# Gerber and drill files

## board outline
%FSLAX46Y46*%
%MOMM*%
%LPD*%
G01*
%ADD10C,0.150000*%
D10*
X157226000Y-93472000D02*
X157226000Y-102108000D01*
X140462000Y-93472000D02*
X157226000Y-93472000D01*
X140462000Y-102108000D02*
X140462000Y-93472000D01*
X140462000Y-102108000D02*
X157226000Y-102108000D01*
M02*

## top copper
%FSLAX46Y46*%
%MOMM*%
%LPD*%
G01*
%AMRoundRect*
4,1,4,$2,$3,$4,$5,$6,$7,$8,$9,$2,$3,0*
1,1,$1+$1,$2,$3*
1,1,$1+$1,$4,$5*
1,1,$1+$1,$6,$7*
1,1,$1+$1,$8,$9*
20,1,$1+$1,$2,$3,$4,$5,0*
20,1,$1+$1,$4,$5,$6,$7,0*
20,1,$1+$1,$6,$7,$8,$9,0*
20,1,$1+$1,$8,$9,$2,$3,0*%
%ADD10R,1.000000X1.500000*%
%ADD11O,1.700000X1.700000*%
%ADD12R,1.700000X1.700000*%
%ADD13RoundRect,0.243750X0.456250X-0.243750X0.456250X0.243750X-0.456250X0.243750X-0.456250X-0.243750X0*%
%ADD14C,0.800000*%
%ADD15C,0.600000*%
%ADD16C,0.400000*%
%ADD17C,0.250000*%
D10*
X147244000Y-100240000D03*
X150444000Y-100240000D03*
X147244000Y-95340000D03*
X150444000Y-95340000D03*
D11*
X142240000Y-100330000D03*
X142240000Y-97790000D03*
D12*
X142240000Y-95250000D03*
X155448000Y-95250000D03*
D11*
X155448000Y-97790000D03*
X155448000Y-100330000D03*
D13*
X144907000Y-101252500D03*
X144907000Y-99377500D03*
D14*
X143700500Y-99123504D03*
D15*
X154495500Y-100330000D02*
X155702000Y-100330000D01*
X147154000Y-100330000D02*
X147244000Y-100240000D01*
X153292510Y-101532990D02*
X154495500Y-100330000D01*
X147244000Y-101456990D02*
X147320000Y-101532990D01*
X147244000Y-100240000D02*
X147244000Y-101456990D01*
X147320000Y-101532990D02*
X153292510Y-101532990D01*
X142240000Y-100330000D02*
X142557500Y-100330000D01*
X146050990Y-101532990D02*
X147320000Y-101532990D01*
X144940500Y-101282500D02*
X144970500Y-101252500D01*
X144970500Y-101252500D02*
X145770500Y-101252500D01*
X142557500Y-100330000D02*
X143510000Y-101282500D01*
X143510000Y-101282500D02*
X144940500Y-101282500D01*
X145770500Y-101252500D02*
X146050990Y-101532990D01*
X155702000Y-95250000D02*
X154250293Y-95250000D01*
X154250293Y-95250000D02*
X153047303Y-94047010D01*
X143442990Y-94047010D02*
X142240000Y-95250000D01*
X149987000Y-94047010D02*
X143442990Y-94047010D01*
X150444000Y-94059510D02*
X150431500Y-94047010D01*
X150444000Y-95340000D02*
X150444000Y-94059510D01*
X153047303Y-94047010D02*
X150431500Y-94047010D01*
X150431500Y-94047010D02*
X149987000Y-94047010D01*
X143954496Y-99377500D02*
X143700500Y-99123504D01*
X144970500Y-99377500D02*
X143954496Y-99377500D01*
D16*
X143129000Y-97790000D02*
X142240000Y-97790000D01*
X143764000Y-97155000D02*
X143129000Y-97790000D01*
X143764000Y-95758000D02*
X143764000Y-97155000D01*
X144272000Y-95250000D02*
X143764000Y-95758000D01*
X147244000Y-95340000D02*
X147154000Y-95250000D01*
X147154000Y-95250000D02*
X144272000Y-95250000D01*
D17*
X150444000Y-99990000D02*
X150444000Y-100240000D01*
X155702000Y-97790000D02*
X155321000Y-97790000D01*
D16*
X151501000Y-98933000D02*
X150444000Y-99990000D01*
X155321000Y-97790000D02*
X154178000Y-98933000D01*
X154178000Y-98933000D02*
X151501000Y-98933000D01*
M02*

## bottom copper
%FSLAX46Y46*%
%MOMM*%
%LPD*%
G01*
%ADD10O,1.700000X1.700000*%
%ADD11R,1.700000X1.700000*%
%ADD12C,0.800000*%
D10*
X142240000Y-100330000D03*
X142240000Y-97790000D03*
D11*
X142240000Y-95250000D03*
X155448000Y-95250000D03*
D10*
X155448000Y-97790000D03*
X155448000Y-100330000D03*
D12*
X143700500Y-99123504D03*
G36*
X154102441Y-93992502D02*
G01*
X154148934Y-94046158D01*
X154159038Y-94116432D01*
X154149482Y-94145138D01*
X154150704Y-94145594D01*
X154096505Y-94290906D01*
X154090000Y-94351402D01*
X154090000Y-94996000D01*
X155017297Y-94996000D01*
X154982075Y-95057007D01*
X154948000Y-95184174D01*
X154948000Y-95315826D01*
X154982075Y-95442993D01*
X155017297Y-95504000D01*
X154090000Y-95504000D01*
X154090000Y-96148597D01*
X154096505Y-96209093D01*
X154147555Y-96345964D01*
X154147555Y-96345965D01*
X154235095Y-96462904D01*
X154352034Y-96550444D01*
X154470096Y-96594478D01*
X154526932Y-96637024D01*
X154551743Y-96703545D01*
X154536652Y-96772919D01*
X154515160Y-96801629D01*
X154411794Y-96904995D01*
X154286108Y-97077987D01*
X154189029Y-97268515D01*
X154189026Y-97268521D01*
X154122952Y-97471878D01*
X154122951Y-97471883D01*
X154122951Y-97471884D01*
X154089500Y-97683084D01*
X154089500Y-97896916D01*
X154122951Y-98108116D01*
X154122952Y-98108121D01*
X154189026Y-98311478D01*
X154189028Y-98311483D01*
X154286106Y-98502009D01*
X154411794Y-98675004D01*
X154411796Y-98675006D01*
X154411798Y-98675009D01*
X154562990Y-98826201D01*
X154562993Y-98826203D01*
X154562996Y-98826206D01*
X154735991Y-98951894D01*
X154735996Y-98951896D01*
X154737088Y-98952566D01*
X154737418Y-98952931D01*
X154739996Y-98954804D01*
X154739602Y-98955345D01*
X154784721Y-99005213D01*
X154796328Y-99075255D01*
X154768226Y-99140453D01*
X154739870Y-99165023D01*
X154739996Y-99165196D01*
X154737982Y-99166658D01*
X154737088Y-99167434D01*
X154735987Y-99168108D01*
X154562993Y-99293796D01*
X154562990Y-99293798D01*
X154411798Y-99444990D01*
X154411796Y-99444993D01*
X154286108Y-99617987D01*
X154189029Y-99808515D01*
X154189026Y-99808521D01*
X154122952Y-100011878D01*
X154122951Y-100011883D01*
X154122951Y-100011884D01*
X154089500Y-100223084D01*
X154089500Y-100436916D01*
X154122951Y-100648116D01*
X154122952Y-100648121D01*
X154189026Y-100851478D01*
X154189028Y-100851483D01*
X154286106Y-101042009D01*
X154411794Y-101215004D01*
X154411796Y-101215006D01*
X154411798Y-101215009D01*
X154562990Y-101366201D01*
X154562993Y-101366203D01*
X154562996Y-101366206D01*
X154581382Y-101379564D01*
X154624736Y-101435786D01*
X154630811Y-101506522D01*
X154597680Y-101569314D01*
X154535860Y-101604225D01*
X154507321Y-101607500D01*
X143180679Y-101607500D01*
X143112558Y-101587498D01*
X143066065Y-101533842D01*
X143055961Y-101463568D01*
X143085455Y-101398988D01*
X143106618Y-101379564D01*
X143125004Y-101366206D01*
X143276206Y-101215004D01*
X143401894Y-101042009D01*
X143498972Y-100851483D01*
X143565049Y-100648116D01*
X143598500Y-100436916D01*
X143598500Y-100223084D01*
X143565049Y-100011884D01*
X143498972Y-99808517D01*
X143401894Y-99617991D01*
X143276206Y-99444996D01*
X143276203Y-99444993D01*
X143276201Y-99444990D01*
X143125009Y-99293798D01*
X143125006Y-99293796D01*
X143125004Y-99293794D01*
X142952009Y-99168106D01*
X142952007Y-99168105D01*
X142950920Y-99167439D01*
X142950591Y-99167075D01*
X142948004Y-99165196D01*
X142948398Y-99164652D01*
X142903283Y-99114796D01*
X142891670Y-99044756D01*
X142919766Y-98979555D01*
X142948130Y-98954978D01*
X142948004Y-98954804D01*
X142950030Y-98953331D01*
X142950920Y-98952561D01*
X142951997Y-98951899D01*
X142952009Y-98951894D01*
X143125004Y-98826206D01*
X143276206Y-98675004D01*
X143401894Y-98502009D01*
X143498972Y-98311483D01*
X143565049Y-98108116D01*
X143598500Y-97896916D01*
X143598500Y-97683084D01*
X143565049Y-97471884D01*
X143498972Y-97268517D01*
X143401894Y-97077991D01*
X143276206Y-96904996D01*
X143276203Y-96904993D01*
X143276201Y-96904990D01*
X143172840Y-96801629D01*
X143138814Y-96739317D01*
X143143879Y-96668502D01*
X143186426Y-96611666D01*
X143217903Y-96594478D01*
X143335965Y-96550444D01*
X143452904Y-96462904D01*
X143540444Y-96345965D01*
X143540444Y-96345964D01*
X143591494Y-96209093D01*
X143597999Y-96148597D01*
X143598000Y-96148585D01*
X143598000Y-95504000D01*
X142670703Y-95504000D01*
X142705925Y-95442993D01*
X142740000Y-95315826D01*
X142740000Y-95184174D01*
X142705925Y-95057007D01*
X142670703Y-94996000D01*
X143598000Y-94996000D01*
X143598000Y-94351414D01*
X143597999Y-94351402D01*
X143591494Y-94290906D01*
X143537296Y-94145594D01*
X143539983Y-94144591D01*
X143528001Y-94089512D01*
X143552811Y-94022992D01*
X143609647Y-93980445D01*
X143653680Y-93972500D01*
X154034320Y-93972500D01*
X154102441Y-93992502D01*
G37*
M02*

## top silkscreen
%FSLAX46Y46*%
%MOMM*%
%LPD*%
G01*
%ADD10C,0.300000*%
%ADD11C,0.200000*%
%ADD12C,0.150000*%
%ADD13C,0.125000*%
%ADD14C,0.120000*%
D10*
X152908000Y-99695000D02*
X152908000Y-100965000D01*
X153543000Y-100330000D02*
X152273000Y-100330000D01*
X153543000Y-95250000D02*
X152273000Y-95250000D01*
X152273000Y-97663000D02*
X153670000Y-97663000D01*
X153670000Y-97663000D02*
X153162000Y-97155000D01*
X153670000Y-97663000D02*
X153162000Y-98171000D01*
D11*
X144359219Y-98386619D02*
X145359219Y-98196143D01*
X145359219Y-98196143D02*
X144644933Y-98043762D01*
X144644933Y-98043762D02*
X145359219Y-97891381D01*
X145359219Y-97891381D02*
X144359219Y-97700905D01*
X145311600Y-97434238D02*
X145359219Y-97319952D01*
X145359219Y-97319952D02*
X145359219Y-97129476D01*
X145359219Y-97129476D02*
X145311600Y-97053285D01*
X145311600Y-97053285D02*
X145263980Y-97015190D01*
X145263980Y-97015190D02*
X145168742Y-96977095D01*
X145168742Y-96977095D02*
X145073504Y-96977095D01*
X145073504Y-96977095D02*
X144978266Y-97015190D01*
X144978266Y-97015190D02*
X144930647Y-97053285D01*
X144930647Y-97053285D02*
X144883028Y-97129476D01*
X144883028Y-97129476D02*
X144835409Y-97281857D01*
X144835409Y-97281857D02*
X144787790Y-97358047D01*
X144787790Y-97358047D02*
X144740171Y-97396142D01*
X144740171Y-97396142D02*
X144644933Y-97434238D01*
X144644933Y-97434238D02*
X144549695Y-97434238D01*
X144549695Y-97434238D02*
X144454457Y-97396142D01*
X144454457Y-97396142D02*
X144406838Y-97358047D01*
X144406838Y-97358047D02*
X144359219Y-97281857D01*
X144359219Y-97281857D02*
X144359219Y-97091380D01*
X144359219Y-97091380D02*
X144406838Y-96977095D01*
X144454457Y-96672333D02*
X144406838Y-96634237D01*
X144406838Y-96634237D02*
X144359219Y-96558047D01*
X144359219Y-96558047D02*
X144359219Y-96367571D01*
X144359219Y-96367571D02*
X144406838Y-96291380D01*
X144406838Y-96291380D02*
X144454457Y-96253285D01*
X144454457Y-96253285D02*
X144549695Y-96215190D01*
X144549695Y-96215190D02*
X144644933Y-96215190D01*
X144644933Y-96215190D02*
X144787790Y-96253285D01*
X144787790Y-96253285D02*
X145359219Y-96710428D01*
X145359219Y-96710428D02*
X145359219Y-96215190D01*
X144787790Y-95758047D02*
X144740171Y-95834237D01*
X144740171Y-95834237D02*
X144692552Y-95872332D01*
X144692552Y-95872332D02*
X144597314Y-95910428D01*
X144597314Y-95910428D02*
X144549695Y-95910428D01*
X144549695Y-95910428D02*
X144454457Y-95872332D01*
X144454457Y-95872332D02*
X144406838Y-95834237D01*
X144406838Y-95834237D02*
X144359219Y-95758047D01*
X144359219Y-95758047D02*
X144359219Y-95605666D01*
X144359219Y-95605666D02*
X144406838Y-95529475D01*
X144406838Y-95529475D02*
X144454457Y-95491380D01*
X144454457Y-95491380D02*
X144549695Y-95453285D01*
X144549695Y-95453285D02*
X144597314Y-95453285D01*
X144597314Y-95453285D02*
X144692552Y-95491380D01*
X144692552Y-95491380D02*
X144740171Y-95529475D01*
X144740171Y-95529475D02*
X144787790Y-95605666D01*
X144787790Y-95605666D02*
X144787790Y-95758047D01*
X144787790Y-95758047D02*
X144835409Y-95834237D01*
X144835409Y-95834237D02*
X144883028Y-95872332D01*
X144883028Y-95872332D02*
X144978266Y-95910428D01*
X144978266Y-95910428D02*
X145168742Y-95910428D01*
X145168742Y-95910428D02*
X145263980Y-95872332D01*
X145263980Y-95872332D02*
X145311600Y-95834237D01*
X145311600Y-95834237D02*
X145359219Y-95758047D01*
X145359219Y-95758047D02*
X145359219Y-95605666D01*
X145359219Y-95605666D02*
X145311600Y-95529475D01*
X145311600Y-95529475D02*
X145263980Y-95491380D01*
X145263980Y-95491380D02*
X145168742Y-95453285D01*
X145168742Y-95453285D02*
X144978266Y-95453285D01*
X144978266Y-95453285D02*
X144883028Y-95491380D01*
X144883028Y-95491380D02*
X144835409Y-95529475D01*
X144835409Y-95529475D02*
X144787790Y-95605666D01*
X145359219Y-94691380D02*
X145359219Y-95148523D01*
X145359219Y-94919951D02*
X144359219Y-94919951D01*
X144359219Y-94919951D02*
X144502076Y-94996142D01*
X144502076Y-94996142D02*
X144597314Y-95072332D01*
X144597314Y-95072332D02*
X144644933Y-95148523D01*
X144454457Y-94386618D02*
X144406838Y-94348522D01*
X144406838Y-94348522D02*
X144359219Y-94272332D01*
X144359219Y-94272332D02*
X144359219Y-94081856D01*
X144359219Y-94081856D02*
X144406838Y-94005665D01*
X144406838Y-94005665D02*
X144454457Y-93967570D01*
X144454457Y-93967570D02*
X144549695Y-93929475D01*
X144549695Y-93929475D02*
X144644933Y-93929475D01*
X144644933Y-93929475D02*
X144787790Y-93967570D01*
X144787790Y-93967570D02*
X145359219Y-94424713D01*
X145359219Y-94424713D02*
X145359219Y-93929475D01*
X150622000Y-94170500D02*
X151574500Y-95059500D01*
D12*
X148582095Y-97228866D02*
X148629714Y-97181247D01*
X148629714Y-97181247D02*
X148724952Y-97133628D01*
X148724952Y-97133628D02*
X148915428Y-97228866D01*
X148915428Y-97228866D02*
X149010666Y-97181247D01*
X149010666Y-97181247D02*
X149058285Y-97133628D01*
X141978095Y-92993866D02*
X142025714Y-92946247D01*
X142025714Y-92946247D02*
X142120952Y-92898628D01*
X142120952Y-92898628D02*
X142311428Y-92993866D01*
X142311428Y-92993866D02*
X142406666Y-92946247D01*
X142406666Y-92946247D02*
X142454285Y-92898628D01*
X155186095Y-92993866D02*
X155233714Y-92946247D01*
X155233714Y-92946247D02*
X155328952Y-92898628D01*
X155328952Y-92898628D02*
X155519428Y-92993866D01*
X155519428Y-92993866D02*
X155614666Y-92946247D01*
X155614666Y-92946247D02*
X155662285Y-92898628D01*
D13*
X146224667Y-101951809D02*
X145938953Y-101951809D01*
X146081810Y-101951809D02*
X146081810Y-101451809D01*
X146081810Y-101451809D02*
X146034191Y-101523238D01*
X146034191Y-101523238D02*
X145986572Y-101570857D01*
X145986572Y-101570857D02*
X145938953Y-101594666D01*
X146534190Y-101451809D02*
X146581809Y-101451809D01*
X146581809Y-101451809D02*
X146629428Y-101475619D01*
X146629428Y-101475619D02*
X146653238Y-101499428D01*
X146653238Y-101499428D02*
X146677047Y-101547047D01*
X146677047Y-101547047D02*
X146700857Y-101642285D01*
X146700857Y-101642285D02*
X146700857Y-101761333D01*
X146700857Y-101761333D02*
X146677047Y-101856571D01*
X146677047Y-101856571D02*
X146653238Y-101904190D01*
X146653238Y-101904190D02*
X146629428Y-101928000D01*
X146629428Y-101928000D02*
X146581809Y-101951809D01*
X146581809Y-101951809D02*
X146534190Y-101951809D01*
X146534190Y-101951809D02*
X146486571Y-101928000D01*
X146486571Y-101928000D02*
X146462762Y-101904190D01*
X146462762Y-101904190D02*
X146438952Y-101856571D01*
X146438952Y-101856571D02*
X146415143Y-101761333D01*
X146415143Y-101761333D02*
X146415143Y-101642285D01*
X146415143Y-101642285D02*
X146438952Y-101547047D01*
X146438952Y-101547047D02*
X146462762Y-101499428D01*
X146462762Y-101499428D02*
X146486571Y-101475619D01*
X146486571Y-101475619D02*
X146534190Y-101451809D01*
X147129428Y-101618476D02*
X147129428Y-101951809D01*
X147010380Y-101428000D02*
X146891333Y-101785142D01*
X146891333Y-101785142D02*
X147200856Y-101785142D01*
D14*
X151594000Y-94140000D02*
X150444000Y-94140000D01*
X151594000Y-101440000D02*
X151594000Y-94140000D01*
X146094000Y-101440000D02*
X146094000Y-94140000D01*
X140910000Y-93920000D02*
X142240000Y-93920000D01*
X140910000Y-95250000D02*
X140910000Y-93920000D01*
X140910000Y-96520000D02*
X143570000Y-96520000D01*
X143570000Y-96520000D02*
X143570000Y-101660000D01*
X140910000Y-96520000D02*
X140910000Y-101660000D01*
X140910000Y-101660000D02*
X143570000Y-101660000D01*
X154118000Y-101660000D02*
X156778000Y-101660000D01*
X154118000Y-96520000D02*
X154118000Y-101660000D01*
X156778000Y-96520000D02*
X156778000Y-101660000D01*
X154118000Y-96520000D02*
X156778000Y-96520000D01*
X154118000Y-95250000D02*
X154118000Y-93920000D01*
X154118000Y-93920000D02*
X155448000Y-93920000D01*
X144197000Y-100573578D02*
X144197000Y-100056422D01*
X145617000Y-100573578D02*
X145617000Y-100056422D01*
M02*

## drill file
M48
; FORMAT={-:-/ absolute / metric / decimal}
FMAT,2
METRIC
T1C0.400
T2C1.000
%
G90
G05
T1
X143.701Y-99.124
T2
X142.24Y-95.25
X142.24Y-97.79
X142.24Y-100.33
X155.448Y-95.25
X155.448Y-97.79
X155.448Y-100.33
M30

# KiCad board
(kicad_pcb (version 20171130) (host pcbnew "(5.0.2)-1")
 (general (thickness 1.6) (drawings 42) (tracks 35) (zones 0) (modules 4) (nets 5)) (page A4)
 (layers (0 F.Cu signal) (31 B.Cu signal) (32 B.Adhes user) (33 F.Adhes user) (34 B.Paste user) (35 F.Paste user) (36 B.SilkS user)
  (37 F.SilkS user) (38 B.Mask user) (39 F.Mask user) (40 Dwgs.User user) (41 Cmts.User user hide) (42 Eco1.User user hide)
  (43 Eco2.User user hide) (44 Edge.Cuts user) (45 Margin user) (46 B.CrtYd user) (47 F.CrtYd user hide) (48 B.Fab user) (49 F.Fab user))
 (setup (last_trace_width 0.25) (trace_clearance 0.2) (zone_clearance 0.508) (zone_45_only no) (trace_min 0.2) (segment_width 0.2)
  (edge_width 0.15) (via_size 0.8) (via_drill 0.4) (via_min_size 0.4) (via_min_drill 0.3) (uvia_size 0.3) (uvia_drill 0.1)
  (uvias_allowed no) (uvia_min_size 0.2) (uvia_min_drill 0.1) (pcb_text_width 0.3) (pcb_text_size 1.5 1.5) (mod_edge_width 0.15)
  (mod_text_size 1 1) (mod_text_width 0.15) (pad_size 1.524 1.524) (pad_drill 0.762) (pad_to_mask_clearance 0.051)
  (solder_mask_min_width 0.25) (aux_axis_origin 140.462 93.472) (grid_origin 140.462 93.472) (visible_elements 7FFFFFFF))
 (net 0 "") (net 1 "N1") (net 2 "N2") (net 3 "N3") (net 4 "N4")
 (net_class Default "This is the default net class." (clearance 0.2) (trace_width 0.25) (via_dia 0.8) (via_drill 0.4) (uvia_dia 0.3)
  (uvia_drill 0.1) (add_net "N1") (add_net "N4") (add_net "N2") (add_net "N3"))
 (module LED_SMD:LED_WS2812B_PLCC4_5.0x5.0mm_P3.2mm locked (layer F.Cu) (at 148.844 97.79 90)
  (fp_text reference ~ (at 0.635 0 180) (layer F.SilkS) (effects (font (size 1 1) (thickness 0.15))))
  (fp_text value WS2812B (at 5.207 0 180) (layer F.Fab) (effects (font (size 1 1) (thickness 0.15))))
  (fp_line (start 3.65 2.75) (end 3.65 1.6) (layer F.SilkS) (width 0.12))
  (fp_line (start -3.65 2.75) (end 3.65 2.75) (layer F.SilkS) (width 0.12))
  (fp_line (start -3.65 -2.75) (end 3.65 -2.75) (layer F.SilkS) (width 0.12))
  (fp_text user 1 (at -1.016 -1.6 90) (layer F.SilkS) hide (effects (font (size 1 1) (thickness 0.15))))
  (pad 1 smd rect (at -2.45 -1.6 90) (size 1.5 1) (layers F.Cu F.Paste F.Mask) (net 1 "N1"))
  (pad 2 smd rect (at -2.45 1.6 90) (size 1.5 1) (layers F.Cu F.Paste F.Mask) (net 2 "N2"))
  (pad 4 smd rect (at 2.45 -1.6 90) (size 1.5 1) (layers F.Cu F.Paste F.Mask) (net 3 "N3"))
  (pad 3 smd rect (at 2.45 1.6 90) (size 1.5 1) (layers F.Cu F.Paste F.Mask) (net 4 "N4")))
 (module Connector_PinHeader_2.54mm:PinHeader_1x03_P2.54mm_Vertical (layer F.Cu) (at 142.24 95.25)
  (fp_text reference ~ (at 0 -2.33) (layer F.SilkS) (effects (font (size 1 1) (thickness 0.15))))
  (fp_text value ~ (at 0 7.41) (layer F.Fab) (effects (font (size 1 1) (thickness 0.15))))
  (fp_line (start -1.33 -1.33) (end 0 -1.33) (layer F.SilkS) (width 0.12))
  (fp_line (start -1.33 0) (end -1.33 -1.33) (layer F.SilkS) (width 0.12))
  (fp_line (start -1.33 1.27) (end 1.33 1.27) (layer F.SilkS) (width 0.12))
  (fp_line (start 1.33 1.27) (end 1.33 6.41) (layer F.SilkS) (width 0.12))
  (fp_line (start -1.33 1.27) (end -1.33 6.41) (layer F.SilkS) (width 0.12))
  (fp_line (start -1.33 6.41) (end 1.33 6.41) (layer F.SilkS) (width 0.12))
  (pad 3 thru_hole oval (at 0 5.08) (size 1.7 1.7) (drill 1) (layers *.Cu *.Mask) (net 1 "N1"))
  (pad 2 thru_hole oval (at 0 2.54) (size 1.7 1.7) (drill 1) (layers *.Cu *.Mask) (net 3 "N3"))
  (pad 1 thru_hole rect (at 0 0) (size 1.7 1.7) (drill 1) (layers *.Cu *.Mask) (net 4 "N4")))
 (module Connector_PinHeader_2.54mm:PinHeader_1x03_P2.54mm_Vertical (layer F.Cu) (at 155.448 95.25)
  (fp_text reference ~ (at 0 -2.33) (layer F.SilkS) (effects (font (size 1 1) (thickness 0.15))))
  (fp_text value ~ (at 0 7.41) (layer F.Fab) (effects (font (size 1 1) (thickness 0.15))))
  (fp_line (start -1.33 6.41) (end 1.33 6.41) (layer F.SilkS) (width 0.12))
  (fp_line (start -1.33 1.27) (end -1.33 6.41) (layer F.SilkS) (width 0.12))
  (fp_line (start 1.33 1.27) (end 1.33 6.41) (layer F.SilkS) (width 0.12))
  (fp_line (start -1.33 1.27) (end 1.33 1.27) (layer F.SilkS) (width 0.12))
  (fp_line (start -1.33 0) (end -1.33 -1.33) (layer F.SilkS) (width 0.12))
  (fp_line (start -1.33 -1.33) (end 0 -1.33) (layer F.SilkS) (width 0.12))
  (pad 1 thru_hole rect (at 0 0) (size 1.7 1.7) (drill 1) (layers *.Cu *.Mask) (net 4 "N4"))
  (pad 2 thru_hole oval (at 0 2.54) (size 1.7 1.7) (drill 1) (layers *.Cu *.Mask) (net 2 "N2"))
  (pad 3 thru_hole oval (at 0 5.08) (size 1.7 1.7) (drill 1) (layers *.Cu *.Mask) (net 1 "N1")))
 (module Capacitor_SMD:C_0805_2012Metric (layer F.Cu) (at 144.907 100.315 90)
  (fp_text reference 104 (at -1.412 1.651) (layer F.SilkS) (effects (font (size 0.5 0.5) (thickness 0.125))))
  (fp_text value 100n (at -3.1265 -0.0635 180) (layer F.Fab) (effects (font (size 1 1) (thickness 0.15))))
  (fp_line (start -0.258578 -0.71) (end 0.258578 -0.71) (layer F.SilkS) (width 0.12))
  (fp_line (start -0.258578 0.71) (end 0.258578 0.71) (layer F.SilkS) (width 0.12))
  (pad 1 smd roundrect (at -0.9375 0 90) (size 0.975 1.4) (layers F.Cu F.Paste F.Mask) (roundrect_rratio 0.25) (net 1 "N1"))
  (pad 2 smd roundrect (at 0.9375 0 90) (size 0.975 1.4) (layers F.Cu F.Paste F.Mask) (roundrect_rratio 0.25) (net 4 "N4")))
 (gr_line (start 152.908 99.695) (end 152.908 100.965) (layer F.SilkS) (width 0.3))
 (gr_line (start 153.543 100.33) (end 152.273 100.33) (layer F.SilkS) (width 0.3))
 (gr_line (start 153.543 95.25) (end 152.273 95.25) (layer F.SilkS) (width 0.3))
 (gr_line (start 152.273 97.663) (end 153.67 97.663) (layer F.SilkS) (width 0.3))
 (gr_line (start 153.67 97.663) (end 153.162 97.155) (layer F.SilkS) (width 0.3))
 (gr_line (start 153.67 97.663) (end 153.162 98.171) (layer F.SilkS) (width 0.3))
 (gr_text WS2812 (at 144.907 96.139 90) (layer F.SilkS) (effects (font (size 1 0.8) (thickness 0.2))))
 (gr_line (start 150.622 94.1705) (end 151.5745 95.0595) (layer F.SilkS) (width 0.2))
 (gr_line (start 157.226 93.472) (end 157.226 102.108) (layer Edge.Cuts) (width 0.15))
 (gr_line (start 140.462 93.472) (end 157.226 93.472) (layer Edge.Cuts) (width 0.15))
 (gr_line (start 140.462 102.108) (end 140.462 93.472) (layer Edge.Cuts) (width 0.15))
 (gr_line (start 140.462 102.108) (end 157.226 102.108) (layer Edge.Cuts) (width 0.15))
 (segment (start 154.4955 100.33) (end 155.702 100.33) (width 0.6) (layer F.Cu) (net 1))
 (segment (start 147.154 100.33) (end 147.244 100.24) (width 0.6) (layer F.Cu) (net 1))
 (segment (start 153.29251 101.53299) (end 154.4955 100.33) (width 0.6) (layer F.Cu) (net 1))
 (segment (start 147.244 101.45699) (end 147.32 101.53299) (width 0.6) (layer F.Cu) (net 1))
 (segment (start 147.244 100.24) (end 147.244 101.45699) (width 0.6) (layer F.Cu) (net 1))
 (segment (start 147.32 101.53299) (end 153.29251 101.53299) (width 0.6) (layer F.Cu) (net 1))
 (segment (start 142.24 100.33) (end 142.5575 100.33) (width 0.6) (layer F.Cu) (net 1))
 (segment (start 146.05099 101.53299) (end 147.32 101.53299) (width 0.6) (layer F.Cu) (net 1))
 (segment (start 144.9405 101.2825) (end 144.9705 101.2525) (width 0.6) (layer F.Cu) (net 1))
 (segment (start 144.9705 101.2525) (end 145.7705 101.2525) (width 0.6) (layer F.Cu) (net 1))
 (segment (start 142.5575 100.33) (end 143.51 101.2825) (width 0.6) (layer F.Cu) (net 1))
 (segment (start 143.51 101.2825) (end 144.9405 101.2825) (width 0.6) (layer F.Cu) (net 1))
 (segment (start 145.7705 101.2525) (end 146.05099 101.53299) (width 0.6) (layer F.Cu) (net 1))
 (segment (start 155.702 95.25) (end 154.250293 95.25) (width 0.6) (layer F.Cu) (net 4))
 (segment (start 154.250293 95.25) (end 153.047303 94.04701) (width 0.6) (layer F.Cu) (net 4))
 (segment (start 143.44299 94.04701) (end 142.24 95.25) (width 0.6) (layer F.Cu) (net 4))
 (segment (start 149.987 94.04701) (end 143.44299 94.04701) (width 0.6) (layer F.Cu) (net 4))
 (segment (start 150.444 94.05951) (end 150.4315 94.04701) (width 0.6) (layer F.Cu) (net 4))
 (segment (start 150.444 95.34) (end 150.444 94.05951) (width 0.6) (layer F.Cu) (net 4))
 (segment (start 153.047303 94.04701) (end 150.4315 94.04701) (width 0.6) (layer F.Cu) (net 4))
 (segment (start 150.4315 94.04701) (end 149.987 94.04701) (width 0.6) (layer F.Cu) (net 4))
 (via (at 143.7005 99.123504) (size 0.8) (drill 0.4) (layers F.Cu B.Cu) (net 4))
 (segment (start 143.954496 99.3775) (end 143.7005 99.123504) (width 0.6) (layer F.Cu) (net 4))
 (segment (start 144.9705 99.3775) (end 143.954496 99.3775) (width 0.6) (layer F.Cu) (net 4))
 (segment (start 143.129 97.79) (end 142.24 97.79) (width 0.4) (layer F.Cu) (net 3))
 (segment (start 143.764 97.155) (end 143.129 97.79) (width 0.4) (layer F.Cu) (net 3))
 (segment (start 143.764 95.758) (end 143.764 97.155) (width 0.4) (layer F.Cu) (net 3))
 (segment (start 144.272 95.25) (end 143.764 95.758) (width 0.4) (layer F.Cu) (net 3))
 (segment (start 147.244 95.34) (end 147.154 95.25) (width 0.4) (layer F.Cu) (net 3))
 (segment (start 147.154 95.25) (end 144.272 95.25) (width 0.4) (layer F.Cu) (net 3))
 (segment (start 150.444 99.99) (end 150.444 100.24) (width 0.25) (layer F.Cu) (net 2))
 (segment (start 155.702 97.79) (end 155.321 97.79) (width 0.25) (layer F.Cu) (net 2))
 (segment (start 151.501 98.933) (end 150.444 99.99) (width 0.4) (layer F.Cu) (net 2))
 (segment (start 155.321 97.79) (end 154.178 98.933) (width 0.4) (layer F.Cu) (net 2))
 (segment (start 154.178 98.933) (end 151.501 98.933) (width 0.4) (layer F.Cu) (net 2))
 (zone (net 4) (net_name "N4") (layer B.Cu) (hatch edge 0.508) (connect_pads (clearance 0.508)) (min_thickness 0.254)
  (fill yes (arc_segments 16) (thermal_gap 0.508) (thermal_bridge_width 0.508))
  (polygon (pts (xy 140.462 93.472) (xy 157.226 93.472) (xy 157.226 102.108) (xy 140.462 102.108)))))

